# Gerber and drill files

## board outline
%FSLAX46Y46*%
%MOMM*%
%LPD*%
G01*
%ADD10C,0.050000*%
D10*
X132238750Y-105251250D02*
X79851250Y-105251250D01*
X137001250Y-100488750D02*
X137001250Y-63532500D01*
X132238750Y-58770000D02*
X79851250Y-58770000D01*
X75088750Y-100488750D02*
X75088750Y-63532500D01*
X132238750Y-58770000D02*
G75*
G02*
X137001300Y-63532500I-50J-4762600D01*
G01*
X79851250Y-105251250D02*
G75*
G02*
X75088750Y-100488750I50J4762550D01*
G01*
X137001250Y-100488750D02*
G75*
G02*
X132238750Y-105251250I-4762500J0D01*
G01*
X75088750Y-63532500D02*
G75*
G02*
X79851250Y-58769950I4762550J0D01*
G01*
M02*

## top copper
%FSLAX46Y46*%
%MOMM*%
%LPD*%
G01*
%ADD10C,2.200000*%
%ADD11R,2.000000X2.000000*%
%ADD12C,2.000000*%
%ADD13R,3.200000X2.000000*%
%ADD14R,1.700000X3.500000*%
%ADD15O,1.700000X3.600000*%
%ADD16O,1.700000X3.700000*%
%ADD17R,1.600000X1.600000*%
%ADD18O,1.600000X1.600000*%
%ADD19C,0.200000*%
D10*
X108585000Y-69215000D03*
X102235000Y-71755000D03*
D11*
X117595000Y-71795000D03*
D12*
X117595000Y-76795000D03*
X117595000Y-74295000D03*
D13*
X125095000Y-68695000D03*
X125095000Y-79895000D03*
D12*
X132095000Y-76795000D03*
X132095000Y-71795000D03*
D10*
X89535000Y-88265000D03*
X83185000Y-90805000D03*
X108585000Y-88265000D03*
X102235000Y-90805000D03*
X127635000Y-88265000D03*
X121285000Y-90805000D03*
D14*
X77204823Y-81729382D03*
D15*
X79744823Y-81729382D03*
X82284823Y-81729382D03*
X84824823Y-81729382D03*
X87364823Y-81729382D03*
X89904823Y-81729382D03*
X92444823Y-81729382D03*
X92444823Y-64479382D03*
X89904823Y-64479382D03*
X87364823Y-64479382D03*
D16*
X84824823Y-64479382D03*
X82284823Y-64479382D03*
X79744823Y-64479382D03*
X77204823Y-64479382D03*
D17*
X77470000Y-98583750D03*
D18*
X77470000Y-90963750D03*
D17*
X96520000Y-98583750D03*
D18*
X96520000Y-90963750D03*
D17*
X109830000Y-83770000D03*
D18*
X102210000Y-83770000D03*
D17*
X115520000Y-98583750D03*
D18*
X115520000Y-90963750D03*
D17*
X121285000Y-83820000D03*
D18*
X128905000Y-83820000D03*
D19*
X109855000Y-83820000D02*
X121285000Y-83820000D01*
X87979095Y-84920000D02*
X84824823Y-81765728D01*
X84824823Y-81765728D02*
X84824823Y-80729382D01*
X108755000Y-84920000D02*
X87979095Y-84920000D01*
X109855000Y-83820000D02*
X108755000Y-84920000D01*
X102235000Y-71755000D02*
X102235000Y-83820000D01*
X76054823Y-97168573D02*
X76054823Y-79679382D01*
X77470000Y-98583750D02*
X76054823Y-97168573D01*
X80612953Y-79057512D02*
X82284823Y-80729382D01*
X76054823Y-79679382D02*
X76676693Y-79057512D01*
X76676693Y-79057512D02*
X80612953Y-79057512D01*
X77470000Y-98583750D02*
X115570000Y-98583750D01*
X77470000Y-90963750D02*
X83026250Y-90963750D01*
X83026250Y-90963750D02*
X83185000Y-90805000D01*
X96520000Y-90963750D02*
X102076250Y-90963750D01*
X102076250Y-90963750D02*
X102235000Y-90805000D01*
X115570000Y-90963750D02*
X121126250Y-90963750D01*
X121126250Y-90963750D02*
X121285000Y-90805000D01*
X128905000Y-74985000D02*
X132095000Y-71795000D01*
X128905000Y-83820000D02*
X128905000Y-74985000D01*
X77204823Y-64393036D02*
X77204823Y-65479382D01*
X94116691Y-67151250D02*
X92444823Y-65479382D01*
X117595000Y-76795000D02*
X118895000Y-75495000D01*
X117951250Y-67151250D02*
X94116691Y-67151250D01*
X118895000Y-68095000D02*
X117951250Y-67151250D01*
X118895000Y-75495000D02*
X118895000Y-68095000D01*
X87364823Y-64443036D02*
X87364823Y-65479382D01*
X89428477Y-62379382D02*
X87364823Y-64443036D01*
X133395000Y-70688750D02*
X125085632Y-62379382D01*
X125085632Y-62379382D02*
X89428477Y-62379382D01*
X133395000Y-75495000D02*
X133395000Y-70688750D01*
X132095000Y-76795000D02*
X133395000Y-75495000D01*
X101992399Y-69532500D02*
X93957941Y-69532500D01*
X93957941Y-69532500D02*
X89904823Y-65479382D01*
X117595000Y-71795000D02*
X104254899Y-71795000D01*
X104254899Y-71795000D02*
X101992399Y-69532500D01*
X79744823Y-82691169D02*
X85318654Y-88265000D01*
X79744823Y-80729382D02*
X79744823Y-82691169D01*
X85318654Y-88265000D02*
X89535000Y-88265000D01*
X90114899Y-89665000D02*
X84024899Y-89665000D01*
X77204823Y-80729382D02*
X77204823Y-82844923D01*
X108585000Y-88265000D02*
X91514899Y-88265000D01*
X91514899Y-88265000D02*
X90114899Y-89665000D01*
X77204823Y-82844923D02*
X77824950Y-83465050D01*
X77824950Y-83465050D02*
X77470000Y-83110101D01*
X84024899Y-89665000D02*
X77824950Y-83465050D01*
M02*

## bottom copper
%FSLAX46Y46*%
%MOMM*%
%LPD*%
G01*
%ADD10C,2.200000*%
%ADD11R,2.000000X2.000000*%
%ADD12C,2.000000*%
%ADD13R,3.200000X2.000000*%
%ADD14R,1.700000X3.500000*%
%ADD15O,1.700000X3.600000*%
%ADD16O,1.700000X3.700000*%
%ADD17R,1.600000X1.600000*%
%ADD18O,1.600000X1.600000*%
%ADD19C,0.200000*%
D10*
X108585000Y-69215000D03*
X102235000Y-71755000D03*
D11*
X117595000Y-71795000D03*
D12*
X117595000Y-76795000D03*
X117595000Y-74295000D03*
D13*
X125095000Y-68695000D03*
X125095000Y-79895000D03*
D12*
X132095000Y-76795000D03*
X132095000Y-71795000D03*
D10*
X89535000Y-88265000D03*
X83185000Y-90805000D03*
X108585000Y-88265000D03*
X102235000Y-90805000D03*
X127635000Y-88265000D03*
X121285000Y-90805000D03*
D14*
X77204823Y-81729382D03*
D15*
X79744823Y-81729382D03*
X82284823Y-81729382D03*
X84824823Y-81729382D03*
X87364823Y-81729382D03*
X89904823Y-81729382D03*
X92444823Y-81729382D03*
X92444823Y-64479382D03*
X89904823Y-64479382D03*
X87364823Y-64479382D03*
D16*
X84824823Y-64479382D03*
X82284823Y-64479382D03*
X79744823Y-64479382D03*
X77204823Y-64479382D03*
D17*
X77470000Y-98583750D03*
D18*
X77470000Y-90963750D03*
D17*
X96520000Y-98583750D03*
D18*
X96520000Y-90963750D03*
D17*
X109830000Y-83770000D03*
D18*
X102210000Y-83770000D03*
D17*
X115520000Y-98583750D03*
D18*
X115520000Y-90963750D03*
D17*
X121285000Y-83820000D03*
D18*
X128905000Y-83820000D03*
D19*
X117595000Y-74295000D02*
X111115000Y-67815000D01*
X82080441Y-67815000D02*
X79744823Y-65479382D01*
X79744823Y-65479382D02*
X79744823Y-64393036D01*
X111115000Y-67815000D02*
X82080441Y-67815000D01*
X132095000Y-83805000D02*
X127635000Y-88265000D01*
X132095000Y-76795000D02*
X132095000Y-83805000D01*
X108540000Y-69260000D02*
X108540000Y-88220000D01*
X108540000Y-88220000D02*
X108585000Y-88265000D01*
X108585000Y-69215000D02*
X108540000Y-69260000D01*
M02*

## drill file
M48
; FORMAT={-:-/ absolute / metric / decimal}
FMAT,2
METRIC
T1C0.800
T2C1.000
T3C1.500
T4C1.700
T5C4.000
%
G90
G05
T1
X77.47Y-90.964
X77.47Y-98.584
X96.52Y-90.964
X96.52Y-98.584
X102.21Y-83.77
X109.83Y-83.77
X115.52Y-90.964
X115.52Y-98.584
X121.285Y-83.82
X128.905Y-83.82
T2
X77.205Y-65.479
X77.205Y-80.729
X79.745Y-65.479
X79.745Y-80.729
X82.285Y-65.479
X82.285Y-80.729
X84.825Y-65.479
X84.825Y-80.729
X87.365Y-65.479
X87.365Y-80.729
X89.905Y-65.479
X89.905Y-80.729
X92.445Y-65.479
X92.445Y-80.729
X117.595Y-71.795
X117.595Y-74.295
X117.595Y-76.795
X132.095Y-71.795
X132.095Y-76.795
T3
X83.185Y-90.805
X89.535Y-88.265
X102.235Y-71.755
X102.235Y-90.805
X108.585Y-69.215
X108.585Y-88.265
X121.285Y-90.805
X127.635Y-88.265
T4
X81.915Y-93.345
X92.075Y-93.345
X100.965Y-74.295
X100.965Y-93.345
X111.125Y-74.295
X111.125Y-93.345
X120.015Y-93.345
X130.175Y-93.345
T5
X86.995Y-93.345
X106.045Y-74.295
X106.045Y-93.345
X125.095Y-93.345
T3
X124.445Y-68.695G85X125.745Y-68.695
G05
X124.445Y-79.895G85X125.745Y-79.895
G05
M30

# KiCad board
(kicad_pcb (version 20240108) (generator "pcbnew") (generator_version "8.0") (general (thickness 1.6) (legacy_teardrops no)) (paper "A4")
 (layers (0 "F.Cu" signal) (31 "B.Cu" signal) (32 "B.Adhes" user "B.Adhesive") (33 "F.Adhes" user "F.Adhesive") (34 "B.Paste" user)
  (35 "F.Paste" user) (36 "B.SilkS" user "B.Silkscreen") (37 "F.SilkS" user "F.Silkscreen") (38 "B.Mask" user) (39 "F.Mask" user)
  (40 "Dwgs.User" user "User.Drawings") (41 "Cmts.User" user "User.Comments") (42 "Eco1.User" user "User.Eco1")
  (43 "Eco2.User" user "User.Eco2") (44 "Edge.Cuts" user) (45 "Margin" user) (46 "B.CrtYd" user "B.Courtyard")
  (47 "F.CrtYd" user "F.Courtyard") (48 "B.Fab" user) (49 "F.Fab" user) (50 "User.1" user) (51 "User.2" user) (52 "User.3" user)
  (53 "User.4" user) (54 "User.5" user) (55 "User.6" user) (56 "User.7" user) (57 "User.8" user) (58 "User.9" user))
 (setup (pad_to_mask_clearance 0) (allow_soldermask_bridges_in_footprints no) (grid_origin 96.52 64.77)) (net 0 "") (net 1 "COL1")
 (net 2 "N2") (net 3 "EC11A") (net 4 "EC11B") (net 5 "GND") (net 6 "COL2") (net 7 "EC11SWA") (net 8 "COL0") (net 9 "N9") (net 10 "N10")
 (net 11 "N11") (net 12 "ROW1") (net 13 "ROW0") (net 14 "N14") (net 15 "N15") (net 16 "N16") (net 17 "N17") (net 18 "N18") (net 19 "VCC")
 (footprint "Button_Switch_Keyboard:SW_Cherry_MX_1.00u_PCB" (layer "F.Cu") (at 108.585 69.215)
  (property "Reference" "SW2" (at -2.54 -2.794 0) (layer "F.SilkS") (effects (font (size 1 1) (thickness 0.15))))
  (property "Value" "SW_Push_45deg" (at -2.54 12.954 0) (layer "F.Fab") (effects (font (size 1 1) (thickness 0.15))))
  (pad "" np_thru_hole circle (at -7.62 5.08) (size 1.7 1.7) (drill 1.7) (layers "*.Cu" "*.Mask"))
  (pad "" np_thru_hole circle (at -2.54 5.08) (size 4 4) (drill 4) (layers "*.Cu" "*.Mask"))
  (pad "" np_thru_hole circle (at 2.54 5.08) (size 1.7 1.7) (drill 1.7) (layers "*.Cu" "*.Mask"))
  (pad "1" thru_hole circle (at 0 0) (size 2.2 2.2) (drill 1.5) (layers "*.Cu" "*.Mask") (remove_unused_layers no) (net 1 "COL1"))
  (pad "2" thru_hole circle (at -6.35 2.54) (size 2.2 2.2) (drill 1.5) (layers "*.Cu" "*.Mask") (remove_unused_layers no) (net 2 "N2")))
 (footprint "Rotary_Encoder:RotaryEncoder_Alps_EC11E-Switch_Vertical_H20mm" (layer "F.Cu") (at 117.595 71.795)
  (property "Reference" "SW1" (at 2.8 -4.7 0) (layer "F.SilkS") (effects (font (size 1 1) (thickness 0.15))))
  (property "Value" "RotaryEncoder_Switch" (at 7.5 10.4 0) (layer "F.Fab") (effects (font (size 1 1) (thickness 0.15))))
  (pad "A" thru_hole rect (at 0 0) (size 2 2) (drill 1) (layers "*.Cu" "*.Mask") (remove_unused_layers no) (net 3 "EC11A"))
  (pad "B" thru_hole circle (at 0 5) (size 2 2) (drill 1) (layers "*.Cu" "*.Mask") (remove_unused_layers no) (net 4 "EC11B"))
  (pad "C" thru_hole circle (at 0 2.5) (size 2 2) (drill 1) (layers "*.Cu" "*.Mask") (remove_unused_layers no) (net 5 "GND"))
  (pad "MP" thru_hole rect (at 7.5 -3.1) (size 3.2 2) (drill oval 2.8 1.5) (layers "*.Cu" "*.Mask") (remove_unused_layers no))
  (pad "MP" thru_hole rect (at 7.5 8.1) (size 3.2 2) (drill oval 2.8 1.5) (layers "*.Cu" "*.Mask") (remove_unused_layers no))
  (pad "S1" thru_hole circle (at 14.5 5) (size 2 2) (drill 1) (layers "*.Cu" "*.Mask") (remove_unused_layers no) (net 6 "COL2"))
  (pad "S2" thru_hole circle (at 14.5 0) (size 2 2) (drill 1) (layers "*.Cu" "*.Mask") (remove_unused_layers no) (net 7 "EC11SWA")))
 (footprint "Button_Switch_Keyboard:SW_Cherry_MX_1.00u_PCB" (layer "F.Cu") (at 89.535 88.265)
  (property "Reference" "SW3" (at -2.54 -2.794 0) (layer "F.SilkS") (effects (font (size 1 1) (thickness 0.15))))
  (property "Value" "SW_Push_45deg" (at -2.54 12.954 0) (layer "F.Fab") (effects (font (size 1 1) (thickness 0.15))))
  (pad "" np_thru_hole circle (at -7.62 5.08) (size 1.7 1.7) (drill 1.7) (layers "*.Cu" "*.Mask"))
  (pad "" np_thru_hole circle (at -2.54 5.08) (size 4 4) (drill 4) (layers "*.Cu" "*.Mask"))
  (pad "" np_thru_hole circle (at 2.54 5.08) (size 1.7 1.7) (drill 1.7) (layers "*.Cu" "*.Mask"))
  (pad "1" thru_hole circle (at 0 0) (size 2.2 2.2) (drill 1.5) (layers "*.Cu" "*.Mask") (remove_unused_layers no) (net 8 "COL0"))
  (pad "2" thru_hole circle (at -6.35 2.54) (size 2.2 2.2) (drill 1.5) (layers "*.Cu" "*.Mask") (remove_unused_layers no) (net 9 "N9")))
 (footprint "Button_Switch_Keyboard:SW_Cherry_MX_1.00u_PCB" (layer "F.Cu") (at 108.585 88.265)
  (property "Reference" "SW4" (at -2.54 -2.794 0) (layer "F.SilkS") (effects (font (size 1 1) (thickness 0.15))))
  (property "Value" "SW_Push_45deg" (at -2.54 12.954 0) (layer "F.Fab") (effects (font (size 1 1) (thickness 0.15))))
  (pad "" np_thru_hole circle (at -7.62 5.08) (size 1.7 1.7) (drill 1.7) (layers "*.Cu" "*.Mask"))
  (pad "" np_thru_hole circle (at -2.54 5.08) (size 4 4) (drill 4) (layers "*.Cu" "*.Mask"))
  (pad "" np_thru_hole circle (at 2.54 5.08) (size 1.7 1.7) (drill 1.7) (layers "*.Cu" "*.Mask"))
  (pad "1" thru_hole circle (at 0 0) (size 2.2 2.2) (drill 1.5) (layers "*.Cu" "*.Mask") (remove_unused_layers no) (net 1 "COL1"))
  (pad "2" thru_hole circle (at -6.35 2.54) (size 2.2 2.2) (drill 1.5) (layers "*.Cu" "*.Mask") (remove_unused_layers no) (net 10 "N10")))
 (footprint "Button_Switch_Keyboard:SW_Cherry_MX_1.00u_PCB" (layer "F.Cu") (at 127.635 88.265)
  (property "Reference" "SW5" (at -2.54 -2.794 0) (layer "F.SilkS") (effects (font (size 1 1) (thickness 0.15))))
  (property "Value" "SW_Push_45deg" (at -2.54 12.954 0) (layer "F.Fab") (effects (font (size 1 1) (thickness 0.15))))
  (pad "" np_thru_hole circle (at -7.62 5.08) (size 1.7 1.7) (drill 1.7) (layers "*.Cu" "*.Mask"))
  (pad "" np_thru_hole circle (at -2.54 5.08) (size 4 4) (drill 4) (layers "*.Cu" "*.Mask"))
  (pad "" np_thru_hole circle (at 2.54 5.08) (size 1.7 1.7) (drill 1.7) (layers "*.Cu" "*.Mask"))
  (pad "1" thru_hole circle (at 0 0) (size 2.2 2.2) (drill 1.5) (layers "*.Cu" "*.Mask") (remove_unused_layers no) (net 6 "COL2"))
  (pad "2" thru_hole circle (at -6.35 2.54) (size 2.2 2.2) (drill 1.5) (layers "*.Cu" "*.Mask") (remove_unused_layers no) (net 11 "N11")))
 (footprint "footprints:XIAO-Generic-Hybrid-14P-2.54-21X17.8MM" (layer "F.Cu") (at 84.824823 73.104382 90)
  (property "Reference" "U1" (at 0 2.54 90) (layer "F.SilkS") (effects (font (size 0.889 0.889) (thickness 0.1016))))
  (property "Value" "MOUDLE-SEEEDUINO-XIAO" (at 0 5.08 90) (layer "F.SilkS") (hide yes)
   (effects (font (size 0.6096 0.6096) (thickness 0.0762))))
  (pad "1" thru_hole rect (at -7.625 -7.62 90) (size 3.5 1.7) (drill 1 (offset -1 0)) (layers "*.Cu" "*.Mask") (remove_unused_layers no)
   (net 1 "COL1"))
  (pad "2" thru_hole oval (at -7.625 -5.08 90) (size 3.6 1.7) (drill 1 (offset -1 0)) (layers "*.Cu" "*.Mask") (remove_unused_layers no)
   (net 8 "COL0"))
  (pad "3" thru_hole oval (at -7.625 -2.54 90) (size 3.6 1.7) (drill 1 (offset -1 0)) (layers "*.Cu" "*.Mask") (remove_unused_layers no)
   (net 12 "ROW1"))
  (pad "4" thru_hole oval (at -7.625 0 90) (size 3.6 1.7) (drill 1 (offset -1 0)) (layers "*.Cu" "*.Mask") (remove_unused_layers no)
   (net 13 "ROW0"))
  (pad "5" thru_hole oval (at -7.625 2.54 90) (size 3.6 1.7) (drill 1 (offset -1 0)) (layers "*.Cu" "*.Mask") (remove_unused_layers no)
   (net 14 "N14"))
  (pad "6" thru_hole oval (at -7.625 5.08 270) (size 3.6 1.7) (drill 1 (offset 1 0)) (layers "*.Cu" "*.Mask") (remove_unused_layers no)
   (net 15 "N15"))
  (pad "7" thru_hole oval (at -7.625 7.62 90) (size 3.6 1.7) (drill 1 (offset -1 0)) (layers "*.Cu" "*.Mask") (remove_unused_layers no)
   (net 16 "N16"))
  (pad "8" thru_hole oval (at 7.625 7.62 90) (size 3.6 1.7) (drill 1 (offset 1 0)) (layers "*.Cu" "*.Mask") (remove_unused_layers no)
   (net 4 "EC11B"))
  (pad "9" thru_hole oval (at 7.625 5.08 90) (size 3.6 1.7) (drill 1 (offset 1 0)) (layers "*.Cu" "*.Mask") (remove_unused_layers no)
   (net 3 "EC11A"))
  (pad "10" thru_hole oval (at 7.625 2.54 90) (size 3.6 1.7) (drill 1 (offset 1 0)) (layers "*.Cu" "*.Mask") (remove_unused_layers no)
   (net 6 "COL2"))
  (pad "11" thru_hole oval (at 7.625 0 90) (size 3.7 1.7) (drill 1 (offset 1 0)) (layers "*.Cu" "*.Mask") (remove_unused_layers no)
   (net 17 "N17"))
  (pad "12" thru_hole oval (at 7.625 -2.54 90) (size 3.7 1.7) (drill 1 (offset 1 0)) (layers "*.Cu" "*.Mask") (remove_unused_layers no)
   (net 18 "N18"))
  (pad "13" thru_hole oval (at 7.625 -5.08 90) (size 3.7 1.7) (drill 1 (offset 1 0)) (layers "*.Cu" "*.Mask") (remove_unused_layers no)
   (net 5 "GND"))
  (pad "14" thru_hole oval (at 7.625 -7.62 90) (size 3.7 1.7) (drill 1 (offset 1 0)) (layers "*.Cu" "*.Mask") (remove_unused_layers no)
   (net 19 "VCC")))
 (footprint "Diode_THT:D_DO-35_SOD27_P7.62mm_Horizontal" (layer "B.Cu") (at 77.47 98.58375 90)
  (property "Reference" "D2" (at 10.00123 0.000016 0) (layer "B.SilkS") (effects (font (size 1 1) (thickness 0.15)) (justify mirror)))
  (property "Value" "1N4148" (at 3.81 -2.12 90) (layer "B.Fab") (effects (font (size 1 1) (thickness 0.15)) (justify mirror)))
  (pad "1" thru_hole rect (at 0 0 90) (size 1.6 1.6) (drill 0.8) (layers "*.Cu" "*.Mask") (remove_unused_layers no) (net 12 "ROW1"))
  (pad "2" thru_hole oval (at 7.62 0 90) (size 1.6 1.6) (drill 0.8) (layers "*.Cu" "*.Mask") (remove_unused_layers no) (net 9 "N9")))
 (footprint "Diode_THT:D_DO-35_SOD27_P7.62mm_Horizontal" (layer "B.Cu") (at 96.52 98.58375 90)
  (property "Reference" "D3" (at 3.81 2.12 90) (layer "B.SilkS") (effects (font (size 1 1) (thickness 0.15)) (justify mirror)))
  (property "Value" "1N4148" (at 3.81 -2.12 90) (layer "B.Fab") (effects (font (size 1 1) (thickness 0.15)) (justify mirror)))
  (pad "1" thru_hole rect (at 0 0 90) (size 1.6 1.6) (drill 0.8) (layers "*.Cu" "*.Mask") (remove_unused_layers no) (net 12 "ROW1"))
  (pad "2" thru_hole oval (at 7.62 0 90) (size 1.6 1.6) (drill 0.8) (layers "*.Cu" "*.Mask") (remove_unused_layers no) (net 10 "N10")))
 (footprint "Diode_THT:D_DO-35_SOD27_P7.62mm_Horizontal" (layer "B.Cu") (at 109.83 83.77 180)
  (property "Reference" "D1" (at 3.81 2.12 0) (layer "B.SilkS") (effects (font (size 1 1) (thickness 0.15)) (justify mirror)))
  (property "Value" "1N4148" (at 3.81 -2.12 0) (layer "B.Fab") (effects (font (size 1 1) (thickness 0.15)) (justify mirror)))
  (pad "1" thru_hole rect (at 0 0 180) (size 1.6 1.6) (drill 0.8) (layers "*.Cu" "*.Mask") (remove_unused_layers no) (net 13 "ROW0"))
  (pad "2" thru_hole oval (at 7.62 0 180) (size 1.6 1.6) (drill 0.8) (layers "*.Cu" "*.Mask") (remove_unused_layers no) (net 2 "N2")))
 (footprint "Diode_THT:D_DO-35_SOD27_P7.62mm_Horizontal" (layer "B.Cu") (at 115.52 98.58375 90)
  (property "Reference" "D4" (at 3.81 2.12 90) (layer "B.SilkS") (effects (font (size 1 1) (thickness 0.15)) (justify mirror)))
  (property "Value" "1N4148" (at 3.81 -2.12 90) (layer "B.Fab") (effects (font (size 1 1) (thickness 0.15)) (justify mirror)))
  (pad "1" thru_hole rect (at 0 0 90) (size 1.6 1.6) (drill 0.8) (layers "*.Cu" "*.Mask") (remove_unused_layers no) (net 12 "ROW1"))
  (pad "2" thru_hole oval (at 7.62 0 90) (size 1.6 1.6) (drill 0.8) (layers "*.Cu" "*.Mask") (remove_unused_layers no) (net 11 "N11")))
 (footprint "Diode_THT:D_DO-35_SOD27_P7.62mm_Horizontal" (layer "B.Cu") (at 121.285 83.82)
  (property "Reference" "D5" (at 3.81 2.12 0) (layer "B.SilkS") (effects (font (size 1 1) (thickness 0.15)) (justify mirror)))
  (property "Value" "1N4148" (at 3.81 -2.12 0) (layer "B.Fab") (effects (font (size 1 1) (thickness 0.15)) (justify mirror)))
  (pad "1" thru_hole rect (at 0 0) (size 1.6 1.6) (drill 0.8) (layers "*.Cu" "*.Mask") (remove_unused_layers no) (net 13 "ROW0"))
  (pad "2" thru_hole oval (at 7.62 0) (size 1.6 1.6) (drill 0.8) (layers "*.Cu" "*.Mask") (remove_unused_layers no) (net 7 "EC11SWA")))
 (gr_line (start 132.23875 105.25125) (end 79.85125 105.25125) (stroke (width 0.05) (type default)) (layer "Edge.Cuts"))
 (gr_line (start 137.00125 100.48875) (end 137.00125 63.5325) (stroke (width 0.05) (type default)) (layer "Edge.Cuts"))
 (gr_line (start 132.23875 58.77) (end 79.85125 58.77) (stroke (width 0.05) (type default)) (layer "Edge.Cuts"))
 (gr_line (start 75.08875 100.48875) (end 75.08875 63.5325) (stroke (width 0.05) (type default)) (layer "Edge.Cuts"))
 (gr_arc (start 132.23875 58.77) (mid 135.606331 60.164919) (end 137.00125 63.5325) (stroke (width 0.05) (type default)) (layer "Edge.Cuts"))
 (gr_arc (start 79.85125 105.25125) (mid 76.483654 103.856346) (end 75.08875 100.48875) (stroke (width 0.05) (type default))
  (layer "Edge.Cuts"))
 (gr_arc (start 137.00125 100.48875) (mid 135.606346 103.856346) (end 132.23875 105.25125) (stroke (width 0.05) (type default))
  (layer "Edge.Cuts"))
 (gr_arc (start 75.08875 63.5325) (mid 76.483654 60.164904) (end 79.85125 58.77) (stroke (width 0.05) (type default)) (layer "Edge.Cuts"))
 (segment (start 117.595 74.295) (end 111.115 67.815) (width 0.2) (layer "B.Cu") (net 5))
 (segment (start 82.080441 67.815) (end 79.744823 65.479382) (width 0.2) (layer "B.Cu") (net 5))
 (segment (start 79.744823 65.479382) (end 79.744823 64.393036) (width 0.2) (layer "B.Cu") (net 5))
 (segment (start 111.115 67.815) (end 82.080441 67.815) (width 0.2) (layer "B.Cu") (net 5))
 (segment (start 109.855 83.82) (end 121.285 83.82) (width 0.2) (layer "F.Cu") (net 13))
 (segment (start 87.979095 84.92) (end 84.824823 81.765728) (width 0.2) (layer "F.Cu") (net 13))
 (segment (start 84.824823 81.765728) (end 84.824823 80.729382) (width 0.2) (layer "F.Cu") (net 13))
 (segment (start 108.755 84.92) (end 87.979095 84.92) (width 0.2) (layer "F.Cu") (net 13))
 (segment (start 109.855 83.82) (end 108.755 84.92) (width 0.2) (layer "F.Cu") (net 13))
 (segment (start 102.235 71.755) (end 102.235 83.82) (width 0.2) (layer "F.Cu") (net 2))
 (segment (start 76.054823 97.168573) (end 76.054823 79.679382) (width 0.2) (layer "F.Cu") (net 12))
 (segment (start 77.47 98.58375) (end 76.054823 97.168573) (width 0.2) (layer "F.Cu") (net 12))
 (segment (start 80.612953 79.057512) (end 82.284823 80.729382) (width 0.2) (layer "F.Cu") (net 12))
 (segment (start 76.054823 79.679382) (end 76.676693 79.057512) (width 0.2) (layer "F.Cu") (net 12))
 (segment (start 76.676693 79.057512) (end 80.612953 79.057512) (width 0.2) (layer "F.Cu") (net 12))
 (segment (start 77.47 98.58375) (end 115.57 98.58375) (width 0.2) (layer "F.Cu") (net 12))
 (segment (start 77.47 90.96375) (end 83.02625 90.96375) (width 0.2) (layer "F.Cu") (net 9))
 (segment (start 83.02625 90.96375) (end 83.185 90.805) (width 0.2) (layer "F.Cu") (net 9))
 (segment (start 96.52 90.96375) (end 102.07625 90.96375) (width 0.2) (layer "F.Cu") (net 10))
 (segment (start 102.07625 90.96375) (end 102.235 90.805) (width 0.2) (layer "F.Cu") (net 10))
 (segment (start 115.57 90.96375) (end 121.12625 90.96375) (width 0.2) (layer "F.Cu") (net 11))
 (segment (start 121.12625 90.96375) (end 121.285 90.805) (width 0.2) (layer "F.Cu") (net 11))
 (segment (start 128.905 74.985) (end 132.095 71.795) (width 0.2) (layer "F.Cu") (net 7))
 (segment (start 128.905 83.82) (end 128.905 74.985) (width 0.2) (layer "F.Cu") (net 7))
 (segment (start 77.204823 64.393036) (end 77.204823 65.479382) (width 0.2) (layer "F.Cu") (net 19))
 (segment (start 94.116691 67.15125) (end 92.444823 65.479382) (width 0.2) (layer "F.Cu") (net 4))
 (segment (start 117.595 76.795) (end 118.895 75.495) (width 0.2) (layer "F.Cu") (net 4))
 (segment (start 117.95125 67.15125) (end 94.116691 67.15125) (width 0.2) (layer "F.Cu") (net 4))
 (segment (start 118.895 68.095) (end 117.95125 67.15125) (width 0.2) (layer "F.Cu") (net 4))
 (segment (start 118.895 75.495) (end 118.895 68.095) (width 0.2) (layer "F.Cu") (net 4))
 (segment (start 87.364823 64.443036) (end 87.364823 65.479382) (width 0.2) (layer "F.Cu") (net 6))
 (segment (start 89.428477 62.379382) (end 87.364823 64.443036) (width 0.2) (layer "F.Cu") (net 6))
 (segment (start 133.395 70.68875) (end 125.085632 62.379382) (width 0.2) (layer "F.Cu") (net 6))
 (segment (start 125.085632 62.379382) (end 89.428477 62.379382) (width 0.2) (layer "F.Cu") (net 6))
 (segment (start 133.395 75.495) (end 133.395 70.68875) (width 0.2) (layer "F.Cu") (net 6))
 (segment (start 132.095 76.795) (end 133.395 75.495) (width 0.2) (layer "F.Cu") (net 6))
 (segment (start 132.095 83.805) (end 127.635 88.265) (width 0.2) (layer "B.Cu") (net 6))
 (segment (start 132.095 76.795) (end 132.095 83.805) (width 0.2) (layer "B.Cu") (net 6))
 (segment (start 101.992399 69.5325) (end 93.957941 69.5325) (width 0.2) (layer "F.Cu") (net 3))
 (segment (start 93.957941 69.5325) (end 89.904823 65.479382) (width 0.2) (layer "F.Cu") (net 3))
 (segment (start 117.595 71.795) (end 104.254899 71.795) (width 0.2) (layer "F.Cu") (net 3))
 (segment (start 104.254899 71.795) (end 101.992399 69.5325) (width 0.2) (layer "F.Cu") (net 3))
 (segment (start 79.744823 82.691169) (end 85.318654 88.265) (width 0.2) (layer "F.Cu") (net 8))
 (segment (start 79.744823 80.729382) (end 79.744823 82.691169) (width 0.2) (layer "F.Cu") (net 8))
 (segment (start 85.318654 88.265) (end 89.535 88.265) (width 0.2) (layer "F.Cu") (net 8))
 (segment (start 90.114899 89.665) (end 84.024899 89.665) (width 0.2) (layer "F.Cu") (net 1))
 (segment (start 77.204823 80.729382) (end 77.204823 82.844923) (width 0.2) (layer "F.Cu") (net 1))
 (segment (start 108.585 88.265) (end 91.514899 88.265) (width 0.2) (layer "F.Cu") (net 1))
 (segment (start 91.514899 88.265) (end 90.114899 89.665) (width 0.2) (layer "F.Cu") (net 1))
 (segment (start 77.204823 82.844923) (end 77.82495 83.46505) (width 0.2) (layer "F.Cu") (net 1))
 (segment (start 77.82495 83.46505) (end 77.47 83.110101) (width 0.2) (layer "F.Cu") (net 1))
 (segment (start 84.024899 89.665) (end 77.82495 83.46505) (width 0.2) (layer "F.Cu") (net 1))
 (segment (start 108.54 69.26) (end 108.54 88.22) (width 0.2) (layer "B.Cu") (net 1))
 (segment (start 108.54 88.22) (end 108.585 88.265) (width 0.2) (layer "B.Cu") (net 1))
 (segment (start 108.585 69.215) (end 108.54 69.26) (width 0.2) (layer "B.Cu") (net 1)))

